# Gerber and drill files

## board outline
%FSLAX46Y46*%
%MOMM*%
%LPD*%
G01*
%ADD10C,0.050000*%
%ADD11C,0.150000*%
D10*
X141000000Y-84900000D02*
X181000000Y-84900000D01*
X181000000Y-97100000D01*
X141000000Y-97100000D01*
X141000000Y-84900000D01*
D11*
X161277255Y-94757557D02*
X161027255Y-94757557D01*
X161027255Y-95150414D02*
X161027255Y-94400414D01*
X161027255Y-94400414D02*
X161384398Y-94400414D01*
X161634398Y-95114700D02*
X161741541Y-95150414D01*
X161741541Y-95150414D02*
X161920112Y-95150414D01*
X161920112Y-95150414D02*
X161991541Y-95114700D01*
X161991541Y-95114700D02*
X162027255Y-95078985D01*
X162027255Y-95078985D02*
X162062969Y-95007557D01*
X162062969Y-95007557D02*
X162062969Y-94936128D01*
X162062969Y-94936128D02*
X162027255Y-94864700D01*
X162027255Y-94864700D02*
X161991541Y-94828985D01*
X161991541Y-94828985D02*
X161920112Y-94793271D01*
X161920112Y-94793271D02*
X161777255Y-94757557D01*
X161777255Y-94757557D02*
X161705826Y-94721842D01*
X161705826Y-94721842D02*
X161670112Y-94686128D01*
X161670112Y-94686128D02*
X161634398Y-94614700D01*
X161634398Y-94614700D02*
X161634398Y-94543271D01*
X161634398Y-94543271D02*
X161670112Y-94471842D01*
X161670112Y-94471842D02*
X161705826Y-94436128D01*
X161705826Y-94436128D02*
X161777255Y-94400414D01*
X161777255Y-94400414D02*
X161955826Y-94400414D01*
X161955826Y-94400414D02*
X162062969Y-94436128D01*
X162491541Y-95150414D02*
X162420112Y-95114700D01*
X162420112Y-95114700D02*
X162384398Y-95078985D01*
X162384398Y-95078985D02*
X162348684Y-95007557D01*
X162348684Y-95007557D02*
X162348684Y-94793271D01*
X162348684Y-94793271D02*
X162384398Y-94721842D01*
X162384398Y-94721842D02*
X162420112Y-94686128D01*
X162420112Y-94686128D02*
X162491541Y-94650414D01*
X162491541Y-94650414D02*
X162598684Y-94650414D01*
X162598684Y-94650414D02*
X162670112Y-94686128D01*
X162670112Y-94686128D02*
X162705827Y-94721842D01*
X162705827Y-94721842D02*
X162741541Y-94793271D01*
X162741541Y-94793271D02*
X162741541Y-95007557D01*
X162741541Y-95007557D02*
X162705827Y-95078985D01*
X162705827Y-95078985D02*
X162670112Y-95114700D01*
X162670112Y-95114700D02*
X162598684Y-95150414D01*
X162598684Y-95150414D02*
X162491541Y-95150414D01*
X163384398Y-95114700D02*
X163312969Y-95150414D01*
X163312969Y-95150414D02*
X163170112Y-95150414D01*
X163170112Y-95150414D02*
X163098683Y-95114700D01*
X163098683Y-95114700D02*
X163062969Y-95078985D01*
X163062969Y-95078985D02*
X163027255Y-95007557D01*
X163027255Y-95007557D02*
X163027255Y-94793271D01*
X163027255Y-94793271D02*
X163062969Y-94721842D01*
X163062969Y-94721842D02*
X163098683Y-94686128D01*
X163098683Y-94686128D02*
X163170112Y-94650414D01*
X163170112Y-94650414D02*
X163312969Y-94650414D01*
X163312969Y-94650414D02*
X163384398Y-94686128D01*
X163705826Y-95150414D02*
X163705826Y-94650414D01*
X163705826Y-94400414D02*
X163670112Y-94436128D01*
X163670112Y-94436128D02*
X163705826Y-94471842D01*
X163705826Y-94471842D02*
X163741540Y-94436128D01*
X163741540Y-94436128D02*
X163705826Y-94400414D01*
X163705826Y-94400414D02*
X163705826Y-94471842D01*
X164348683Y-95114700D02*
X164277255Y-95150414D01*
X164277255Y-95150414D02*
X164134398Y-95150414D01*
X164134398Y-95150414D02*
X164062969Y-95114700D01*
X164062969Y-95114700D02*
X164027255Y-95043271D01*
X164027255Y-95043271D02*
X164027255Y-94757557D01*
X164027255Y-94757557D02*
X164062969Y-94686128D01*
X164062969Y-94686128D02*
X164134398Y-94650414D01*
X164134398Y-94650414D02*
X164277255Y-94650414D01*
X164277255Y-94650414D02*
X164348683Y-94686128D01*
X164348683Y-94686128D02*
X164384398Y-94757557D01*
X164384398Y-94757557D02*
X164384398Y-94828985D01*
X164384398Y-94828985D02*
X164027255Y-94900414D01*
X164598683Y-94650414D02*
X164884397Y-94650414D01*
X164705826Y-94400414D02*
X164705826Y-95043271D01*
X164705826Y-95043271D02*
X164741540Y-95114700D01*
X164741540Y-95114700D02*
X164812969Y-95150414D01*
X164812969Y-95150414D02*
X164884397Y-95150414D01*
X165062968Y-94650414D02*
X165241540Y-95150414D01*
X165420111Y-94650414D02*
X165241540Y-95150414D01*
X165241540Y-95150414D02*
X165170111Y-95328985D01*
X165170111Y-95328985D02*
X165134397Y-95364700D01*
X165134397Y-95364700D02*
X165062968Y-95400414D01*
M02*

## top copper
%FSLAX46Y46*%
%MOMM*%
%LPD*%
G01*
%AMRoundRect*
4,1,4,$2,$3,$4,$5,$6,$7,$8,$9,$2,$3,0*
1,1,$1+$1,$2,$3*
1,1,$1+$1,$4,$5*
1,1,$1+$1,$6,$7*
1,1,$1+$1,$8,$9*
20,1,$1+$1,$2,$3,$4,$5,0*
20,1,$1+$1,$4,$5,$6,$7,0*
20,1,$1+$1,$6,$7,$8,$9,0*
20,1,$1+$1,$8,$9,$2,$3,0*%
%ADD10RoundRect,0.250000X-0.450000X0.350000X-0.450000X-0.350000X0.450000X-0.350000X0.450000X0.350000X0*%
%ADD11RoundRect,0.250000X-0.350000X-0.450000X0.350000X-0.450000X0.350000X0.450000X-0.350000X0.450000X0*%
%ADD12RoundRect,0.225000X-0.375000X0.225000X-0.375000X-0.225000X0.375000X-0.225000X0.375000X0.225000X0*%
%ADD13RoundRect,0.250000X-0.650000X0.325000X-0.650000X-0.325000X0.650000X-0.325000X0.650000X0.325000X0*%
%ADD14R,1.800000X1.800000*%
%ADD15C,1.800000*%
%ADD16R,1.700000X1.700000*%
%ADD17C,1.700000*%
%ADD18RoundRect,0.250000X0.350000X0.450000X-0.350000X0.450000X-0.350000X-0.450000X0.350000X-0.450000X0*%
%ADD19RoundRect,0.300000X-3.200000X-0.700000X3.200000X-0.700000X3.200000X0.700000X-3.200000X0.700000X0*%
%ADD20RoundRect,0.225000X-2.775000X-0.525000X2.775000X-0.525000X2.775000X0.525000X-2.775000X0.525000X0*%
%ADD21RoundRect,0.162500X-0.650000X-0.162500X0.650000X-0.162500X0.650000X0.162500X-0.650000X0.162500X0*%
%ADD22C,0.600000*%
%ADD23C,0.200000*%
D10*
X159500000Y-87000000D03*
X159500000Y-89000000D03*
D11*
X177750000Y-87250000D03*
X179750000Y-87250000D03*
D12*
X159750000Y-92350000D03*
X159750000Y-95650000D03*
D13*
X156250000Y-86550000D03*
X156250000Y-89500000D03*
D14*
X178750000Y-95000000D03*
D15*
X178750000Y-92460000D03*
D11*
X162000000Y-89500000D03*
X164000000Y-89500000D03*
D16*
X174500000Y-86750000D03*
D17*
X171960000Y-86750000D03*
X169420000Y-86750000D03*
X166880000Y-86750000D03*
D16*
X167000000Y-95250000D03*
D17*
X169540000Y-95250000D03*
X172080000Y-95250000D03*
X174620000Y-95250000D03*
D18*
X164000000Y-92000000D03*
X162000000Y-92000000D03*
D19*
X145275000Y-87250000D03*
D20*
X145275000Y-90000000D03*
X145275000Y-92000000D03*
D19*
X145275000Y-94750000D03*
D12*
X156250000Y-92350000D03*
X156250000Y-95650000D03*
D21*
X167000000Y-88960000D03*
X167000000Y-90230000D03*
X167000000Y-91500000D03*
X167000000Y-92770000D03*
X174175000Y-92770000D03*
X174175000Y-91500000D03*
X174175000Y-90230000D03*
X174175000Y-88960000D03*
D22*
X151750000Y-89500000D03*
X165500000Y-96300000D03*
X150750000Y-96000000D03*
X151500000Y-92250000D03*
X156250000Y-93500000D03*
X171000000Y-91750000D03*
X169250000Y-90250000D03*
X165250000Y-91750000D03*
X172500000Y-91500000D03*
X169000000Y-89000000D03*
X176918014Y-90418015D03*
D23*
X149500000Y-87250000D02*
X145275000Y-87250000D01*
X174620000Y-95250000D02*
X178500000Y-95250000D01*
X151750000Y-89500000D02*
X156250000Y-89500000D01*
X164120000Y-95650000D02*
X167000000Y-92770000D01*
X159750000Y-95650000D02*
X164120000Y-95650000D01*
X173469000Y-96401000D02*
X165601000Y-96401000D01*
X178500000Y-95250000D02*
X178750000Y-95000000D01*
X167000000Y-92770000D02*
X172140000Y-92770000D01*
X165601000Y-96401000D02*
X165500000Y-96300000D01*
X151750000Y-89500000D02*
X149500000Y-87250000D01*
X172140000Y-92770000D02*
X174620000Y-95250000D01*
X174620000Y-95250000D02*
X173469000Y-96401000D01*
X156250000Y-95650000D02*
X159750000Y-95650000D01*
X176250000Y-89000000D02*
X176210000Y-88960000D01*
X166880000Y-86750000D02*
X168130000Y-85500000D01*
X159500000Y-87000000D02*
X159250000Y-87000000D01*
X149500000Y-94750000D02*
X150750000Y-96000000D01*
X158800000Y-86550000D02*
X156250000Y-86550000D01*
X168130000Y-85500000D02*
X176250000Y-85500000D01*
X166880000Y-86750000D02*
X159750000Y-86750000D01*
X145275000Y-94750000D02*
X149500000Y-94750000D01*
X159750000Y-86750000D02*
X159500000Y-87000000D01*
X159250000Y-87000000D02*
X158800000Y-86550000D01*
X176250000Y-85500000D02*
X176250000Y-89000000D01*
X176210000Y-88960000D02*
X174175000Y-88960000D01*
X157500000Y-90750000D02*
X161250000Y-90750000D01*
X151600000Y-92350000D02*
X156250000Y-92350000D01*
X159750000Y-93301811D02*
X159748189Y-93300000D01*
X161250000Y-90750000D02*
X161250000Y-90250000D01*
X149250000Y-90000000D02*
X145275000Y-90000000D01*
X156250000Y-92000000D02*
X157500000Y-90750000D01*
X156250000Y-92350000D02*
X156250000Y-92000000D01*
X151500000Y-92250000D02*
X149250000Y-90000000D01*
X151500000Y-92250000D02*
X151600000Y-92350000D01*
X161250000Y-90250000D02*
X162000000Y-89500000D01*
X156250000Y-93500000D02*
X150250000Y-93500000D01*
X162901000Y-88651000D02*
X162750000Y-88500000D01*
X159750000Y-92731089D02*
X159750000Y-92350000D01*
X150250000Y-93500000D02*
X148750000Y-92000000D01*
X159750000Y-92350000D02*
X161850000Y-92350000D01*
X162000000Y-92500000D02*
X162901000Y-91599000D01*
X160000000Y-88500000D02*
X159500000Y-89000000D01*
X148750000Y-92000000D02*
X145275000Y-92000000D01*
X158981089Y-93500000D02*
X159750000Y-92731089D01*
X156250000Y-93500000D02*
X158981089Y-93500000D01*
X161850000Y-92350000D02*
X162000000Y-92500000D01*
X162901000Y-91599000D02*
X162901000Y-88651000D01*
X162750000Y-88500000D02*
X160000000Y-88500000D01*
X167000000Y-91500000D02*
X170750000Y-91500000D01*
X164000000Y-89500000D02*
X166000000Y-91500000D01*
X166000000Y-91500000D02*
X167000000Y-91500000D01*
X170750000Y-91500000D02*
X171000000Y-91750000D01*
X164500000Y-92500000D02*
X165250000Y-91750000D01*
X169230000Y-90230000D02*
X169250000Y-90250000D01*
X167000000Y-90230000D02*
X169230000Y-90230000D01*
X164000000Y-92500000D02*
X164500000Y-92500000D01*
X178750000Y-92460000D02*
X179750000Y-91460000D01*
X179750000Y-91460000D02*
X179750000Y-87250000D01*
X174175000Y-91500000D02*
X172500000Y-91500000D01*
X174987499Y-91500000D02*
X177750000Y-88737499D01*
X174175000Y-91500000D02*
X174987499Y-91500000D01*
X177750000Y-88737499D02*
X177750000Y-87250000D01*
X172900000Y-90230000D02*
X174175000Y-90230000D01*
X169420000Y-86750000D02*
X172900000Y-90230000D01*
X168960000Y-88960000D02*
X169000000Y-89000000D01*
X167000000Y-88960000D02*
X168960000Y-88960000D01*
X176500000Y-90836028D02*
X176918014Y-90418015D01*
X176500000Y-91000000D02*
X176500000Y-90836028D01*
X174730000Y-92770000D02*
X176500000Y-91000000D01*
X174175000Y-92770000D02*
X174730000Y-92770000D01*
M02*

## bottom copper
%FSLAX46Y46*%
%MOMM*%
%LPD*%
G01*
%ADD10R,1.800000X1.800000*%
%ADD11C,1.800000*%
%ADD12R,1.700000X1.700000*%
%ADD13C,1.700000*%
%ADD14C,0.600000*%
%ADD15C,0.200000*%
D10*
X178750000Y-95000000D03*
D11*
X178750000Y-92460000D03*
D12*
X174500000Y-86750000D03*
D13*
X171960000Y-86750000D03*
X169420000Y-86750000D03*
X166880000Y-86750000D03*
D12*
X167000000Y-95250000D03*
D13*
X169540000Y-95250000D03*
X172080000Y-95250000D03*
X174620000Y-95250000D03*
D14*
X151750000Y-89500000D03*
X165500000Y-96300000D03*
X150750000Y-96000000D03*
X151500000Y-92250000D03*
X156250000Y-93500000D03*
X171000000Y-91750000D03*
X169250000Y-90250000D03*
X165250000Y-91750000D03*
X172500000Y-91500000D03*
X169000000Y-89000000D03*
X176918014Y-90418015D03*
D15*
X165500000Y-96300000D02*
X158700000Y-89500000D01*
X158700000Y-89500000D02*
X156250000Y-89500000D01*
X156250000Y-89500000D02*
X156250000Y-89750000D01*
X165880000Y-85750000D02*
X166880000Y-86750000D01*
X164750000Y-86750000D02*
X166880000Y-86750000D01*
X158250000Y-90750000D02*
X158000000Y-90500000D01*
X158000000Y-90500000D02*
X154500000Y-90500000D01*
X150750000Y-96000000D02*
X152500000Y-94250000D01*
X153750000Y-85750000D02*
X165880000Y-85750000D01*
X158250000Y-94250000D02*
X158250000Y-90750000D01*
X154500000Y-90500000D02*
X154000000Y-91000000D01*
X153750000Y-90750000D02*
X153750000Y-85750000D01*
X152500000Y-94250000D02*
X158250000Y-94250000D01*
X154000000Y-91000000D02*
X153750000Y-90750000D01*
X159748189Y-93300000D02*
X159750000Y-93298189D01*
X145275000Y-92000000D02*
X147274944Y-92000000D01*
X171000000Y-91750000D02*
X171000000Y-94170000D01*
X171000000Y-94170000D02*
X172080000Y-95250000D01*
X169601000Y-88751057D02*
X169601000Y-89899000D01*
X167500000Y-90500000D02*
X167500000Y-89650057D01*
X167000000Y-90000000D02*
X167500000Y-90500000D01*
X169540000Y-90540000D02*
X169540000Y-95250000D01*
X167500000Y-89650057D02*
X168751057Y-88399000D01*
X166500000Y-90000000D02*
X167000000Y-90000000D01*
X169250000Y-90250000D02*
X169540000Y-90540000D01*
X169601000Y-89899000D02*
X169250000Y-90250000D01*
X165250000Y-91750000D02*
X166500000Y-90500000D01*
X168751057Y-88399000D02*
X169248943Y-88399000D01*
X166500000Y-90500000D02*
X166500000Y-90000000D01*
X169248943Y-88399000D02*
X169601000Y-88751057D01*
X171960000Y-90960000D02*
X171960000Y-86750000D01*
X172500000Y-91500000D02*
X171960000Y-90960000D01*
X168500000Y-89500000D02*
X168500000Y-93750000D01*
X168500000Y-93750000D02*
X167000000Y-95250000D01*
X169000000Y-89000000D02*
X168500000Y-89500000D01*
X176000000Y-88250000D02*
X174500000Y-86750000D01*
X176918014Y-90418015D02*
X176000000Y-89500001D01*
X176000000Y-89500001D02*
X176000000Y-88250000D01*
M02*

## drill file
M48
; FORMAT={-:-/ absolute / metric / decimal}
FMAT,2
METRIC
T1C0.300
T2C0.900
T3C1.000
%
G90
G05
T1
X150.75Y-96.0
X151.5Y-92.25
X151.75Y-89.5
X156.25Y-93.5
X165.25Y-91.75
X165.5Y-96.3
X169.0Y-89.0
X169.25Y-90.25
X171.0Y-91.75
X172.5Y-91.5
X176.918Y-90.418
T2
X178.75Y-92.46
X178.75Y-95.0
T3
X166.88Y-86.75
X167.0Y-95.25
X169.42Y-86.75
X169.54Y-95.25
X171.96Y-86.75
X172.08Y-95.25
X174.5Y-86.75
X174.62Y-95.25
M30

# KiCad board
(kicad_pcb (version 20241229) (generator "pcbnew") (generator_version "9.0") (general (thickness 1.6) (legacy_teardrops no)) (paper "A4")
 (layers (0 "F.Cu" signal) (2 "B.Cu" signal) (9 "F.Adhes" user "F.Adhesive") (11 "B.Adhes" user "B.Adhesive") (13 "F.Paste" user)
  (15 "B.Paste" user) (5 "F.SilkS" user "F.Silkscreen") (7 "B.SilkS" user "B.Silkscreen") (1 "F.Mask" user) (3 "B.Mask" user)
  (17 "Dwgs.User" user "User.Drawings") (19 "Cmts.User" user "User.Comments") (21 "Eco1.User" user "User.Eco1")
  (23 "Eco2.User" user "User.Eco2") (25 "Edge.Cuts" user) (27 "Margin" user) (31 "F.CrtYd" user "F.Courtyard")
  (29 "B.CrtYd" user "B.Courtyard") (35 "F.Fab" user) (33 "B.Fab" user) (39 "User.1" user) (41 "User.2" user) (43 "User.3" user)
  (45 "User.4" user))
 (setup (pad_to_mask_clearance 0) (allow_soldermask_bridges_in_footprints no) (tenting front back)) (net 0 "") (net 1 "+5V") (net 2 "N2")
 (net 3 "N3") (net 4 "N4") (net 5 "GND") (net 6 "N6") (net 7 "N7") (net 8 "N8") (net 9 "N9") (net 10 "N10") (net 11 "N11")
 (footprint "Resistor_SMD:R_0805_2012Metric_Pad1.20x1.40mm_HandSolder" (layer "F.Cu") (at 159.5 88 -90)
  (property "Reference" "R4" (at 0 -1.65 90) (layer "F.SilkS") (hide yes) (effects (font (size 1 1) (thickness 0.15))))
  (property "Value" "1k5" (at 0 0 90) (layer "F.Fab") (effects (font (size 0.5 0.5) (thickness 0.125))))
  (pad "1" smd roundrect (at -1 0 270) (size 1.2 1.4) (layers "F.Cu" "F.Mask" "F.Paste") (roundrect_rratio 0.208333) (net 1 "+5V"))
  (pad "2" smd roundrect (at 1 0 270) (size 1.2 1.4) (layers "F.Cu" "F.Mask" "F.Paste") (roundrect_rratio 0.208333) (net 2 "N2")))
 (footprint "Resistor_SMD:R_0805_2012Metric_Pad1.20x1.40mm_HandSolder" (layer "F.Cu") (at 178.75 87.25)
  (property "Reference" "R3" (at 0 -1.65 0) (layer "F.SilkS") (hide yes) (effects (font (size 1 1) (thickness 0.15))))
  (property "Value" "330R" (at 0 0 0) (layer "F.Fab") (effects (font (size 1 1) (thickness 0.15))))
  (pad "1" smd roundrect (at -1 0) (size 1.2 1.4) (layers "F.Cu" "F.Mask" "F.Paste") (roundrect_rratio 0.208333) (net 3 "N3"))
  (pad "2" smd roundrect (at 1 0) (size 1.2 1.4) (layers "F.Cu" "F.Mask" "F.Paste") (roundrect_rratio 0.208333) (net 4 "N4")))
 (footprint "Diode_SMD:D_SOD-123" (layer "F.Cu") (at 159.75 94 -90)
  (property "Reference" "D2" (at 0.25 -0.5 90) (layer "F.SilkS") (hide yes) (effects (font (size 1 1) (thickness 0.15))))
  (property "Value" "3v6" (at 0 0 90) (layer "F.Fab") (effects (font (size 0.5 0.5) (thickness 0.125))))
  (pad "1" smd roundrect (at -1.65 0 270) (size 0.9 1.2) (layers "F.Cu" "F.Mask" "F.Paste") (roundrect_rratio 0.25) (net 2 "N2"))
  (pad "2" smd roundrect (at 1.65 0 270) (size 0.9 1.2) (layers "F.Cu" "F.Mask" "F.Paste") (roundrect_rratio 0.25) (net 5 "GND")))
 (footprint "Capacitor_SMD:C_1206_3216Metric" (layer "F.Cu") (at 156.25 88.025 -90)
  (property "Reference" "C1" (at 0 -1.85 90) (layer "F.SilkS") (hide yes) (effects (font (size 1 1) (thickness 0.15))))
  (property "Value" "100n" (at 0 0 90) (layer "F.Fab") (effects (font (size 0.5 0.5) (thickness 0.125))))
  (pad "1" smd roundrect (at -1.475 0 270) (size 1.15 1.8) (layers "F.Cu" "F.Mask" "F.Paste") (roundrect_rratio 0.217391) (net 1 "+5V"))
  (pad "2" smd roundrect (at 1.475 0 270) (size 1.15 1.8) (layers "F.Cu" "F.Mask" "F.Paste") (roundrect_rratio 0.217391) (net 5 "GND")))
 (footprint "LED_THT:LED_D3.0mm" (layer "F.Cu") (at 178.75 95 90)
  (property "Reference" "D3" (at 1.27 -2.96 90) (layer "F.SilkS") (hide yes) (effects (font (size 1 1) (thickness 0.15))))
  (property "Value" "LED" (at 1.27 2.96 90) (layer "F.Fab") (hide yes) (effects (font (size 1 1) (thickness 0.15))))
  (pad "1" thru_hole rect (at 0 0 90) (size 1.8 1.8) (drill 0.9) (layers "*.Cu" "*.Mask") (remove_unused_layers no) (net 5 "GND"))
  (pad "2" thru_hole circle (at 2.54 0 90) (size 1.8 1.8) (drill 0.9) (layers "*.Cu" "*.Mask") (remove_unused_layers no) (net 4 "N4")))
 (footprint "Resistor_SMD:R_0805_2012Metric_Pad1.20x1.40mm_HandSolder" (layer "F.Cu") (at 163 89.5)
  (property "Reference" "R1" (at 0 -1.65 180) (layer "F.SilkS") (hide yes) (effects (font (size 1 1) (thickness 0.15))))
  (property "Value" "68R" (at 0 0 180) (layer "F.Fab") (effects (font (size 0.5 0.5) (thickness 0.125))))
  (pad "1" smd roundrect (at -1 0) (size 1.2 1.4) (layers "F.Cu" "F.Mask" "F.Paste") (roundrect_rratio 0.208333) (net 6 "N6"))
  (pad "2" smd roundrect (at 1 0) (size 1.2 1.4) (layers "F.Cu" "F.Mask" "F.Paste") (roundrect_rratio 0.208333) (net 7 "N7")))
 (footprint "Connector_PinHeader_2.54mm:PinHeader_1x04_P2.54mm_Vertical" (layer "F.Cu") (at 174.5 86.75 -90)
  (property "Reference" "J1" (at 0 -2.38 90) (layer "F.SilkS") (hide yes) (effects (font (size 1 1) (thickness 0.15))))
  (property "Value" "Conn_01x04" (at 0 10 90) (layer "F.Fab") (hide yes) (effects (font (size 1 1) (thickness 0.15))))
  (pad "1" thru_hole rect (at 0 0 270) (size 1.7 1.7) (drill 1) (layers "*.Cu" "*.Mask") (remove_unused_layers no) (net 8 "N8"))
  (pad "2" thru_hole circle (at 0 2.54 270) (size 1.7 1.7) (drill 1) (layers "*.Cu" "*.Mask") (remove_unused_layers no) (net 3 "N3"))
  (pad "3" thru_hole circle (at 0 5.08 270) (size 1.7 1.7) (drill 1) (layers "*.Cu" "*.Mask") (remove_unused_layers no) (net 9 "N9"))
  (pad "4" thru_hole circle (at 0 7.62 270) (size 1.7 1.7) (drill 1) (layers "*.Cu" "*.Mask") (remove_unused_layers no) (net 1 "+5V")))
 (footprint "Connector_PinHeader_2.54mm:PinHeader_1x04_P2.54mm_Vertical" (layer "F.Cu") (at 167 95.25 90)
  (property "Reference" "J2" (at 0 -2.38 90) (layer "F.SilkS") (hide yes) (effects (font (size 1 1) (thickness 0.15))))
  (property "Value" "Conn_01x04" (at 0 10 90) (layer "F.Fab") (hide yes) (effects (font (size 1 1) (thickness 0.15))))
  (pad "1" thru_hole rect (at 0 0 90) (size 1.7 1.7) (drill 1) (layers "*.Cu" "*.Mask") (remove_unused_layers no) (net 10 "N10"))
  (pad "2" thru_hole circle (at 0 2.54 90) (size 1.7 1.7) (drill 1) (layers "*.Cu" "*.Mask") (remove_unused_layers no) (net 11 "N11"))
  (pad "3" thru_hole circle (at 0 5.08 90) (size 1.7 1.7) (drill 1) (layers "*.Cu" "*.Mask") (remove_unused_layers no) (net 7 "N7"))
  (pad "4" thru_hole circle (at 0 7.62 90) (size 1.7 1.7) (drill 1) (layers "*.Cu" "*.Mask") (remove_unused_layers no) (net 5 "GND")))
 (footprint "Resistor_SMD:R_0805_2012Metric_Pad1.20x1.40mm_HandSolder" (layer "F.Cu") (at 163 92 180)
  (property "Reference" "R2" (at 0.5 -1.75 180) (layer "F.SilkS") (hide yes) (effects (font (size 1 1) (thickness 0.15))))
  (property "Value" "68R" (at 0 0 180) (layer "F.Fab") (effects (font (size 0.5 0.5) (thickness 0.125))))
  (pad "1" smd roundrect (at -1 0 180) (size 1.2 1.4) (layers "F.Cu" "F.Mask" "F.Paste") (roundrect_rratio 0.208333) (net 11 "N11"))
  (pad "2" smd roundrect (at 1 0 180) (size 1.2 1.4) (layers "F.Cu" "F.Mask" "F.Paste") (roundrect_rratio 0.208333) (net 2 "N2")))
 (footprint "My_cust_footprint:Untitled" (layer "F.Cu") (at 145.275 91)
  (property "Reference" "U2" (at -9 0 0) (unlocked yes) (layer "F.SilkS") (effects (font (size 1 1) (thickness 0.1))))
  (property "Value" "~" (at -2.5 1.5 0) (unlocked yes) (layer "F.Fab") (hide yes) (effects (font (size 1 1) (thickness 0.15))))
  (pad "1" smd roundrect (at 0 -3.75) (size 7 2) (layers "F.Cu" "F.Mask" "F.Paste") (roundrect_rratio 0.15) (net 5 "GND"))
  (pad "2" smd roundrect (at 0 -1) (size 6 1.5) (layers "F.Cu" "F.Mask" "F.Paste") (roundrect_rratio 0.15) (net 6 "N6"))
  (pad "3" smd roundrect (at 0 1) (size 6 1.5) (layers "F.Cu" "F.Mask" "F.Paste") (roundrect_rratio 0.15) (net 2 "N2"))
  (pad "4" smd roundrect (at 0 3.75) (size 7 2) (layers "F.Cu" "F.Mask" "F.Paste") (roundrect_rratio 0.15) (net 1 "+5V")))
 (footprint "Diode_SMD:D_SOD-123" (layer "F.Cu") (at 156.25 94 -90)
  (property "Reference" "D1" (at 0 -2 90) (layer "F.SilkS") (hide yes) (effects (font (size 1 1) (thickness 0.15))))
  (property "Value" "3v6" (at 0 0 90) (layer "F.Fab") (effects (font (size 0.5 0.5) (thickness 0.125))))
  (pad "1" smd roundrect (at -1.65 0 270) (size 0.9 1.2) (layers "F.Cu" "F.Mask" "F.Paste") (roundrect_rratio 0.25) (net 6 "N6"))
  (pad "2" smd roundrect (at 1.65 0 270) (size 0.9 1.2) (layers "F.Cu" "F.Mask" "F.Paste") (roundrect_rratio 0.25) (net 5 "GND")))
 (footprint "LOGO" (layer "F.Cu") (at 152 91.5)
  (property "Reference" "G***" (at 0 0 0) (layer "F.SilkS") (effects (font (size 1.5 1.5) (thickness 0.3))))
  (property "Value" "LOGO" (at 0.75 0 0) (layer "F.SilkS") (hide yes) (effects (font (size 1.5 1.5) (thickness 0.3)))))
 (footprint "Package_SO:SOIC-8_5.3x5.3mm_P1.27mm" (layer "F.Cu") (at 170.5875 90.865)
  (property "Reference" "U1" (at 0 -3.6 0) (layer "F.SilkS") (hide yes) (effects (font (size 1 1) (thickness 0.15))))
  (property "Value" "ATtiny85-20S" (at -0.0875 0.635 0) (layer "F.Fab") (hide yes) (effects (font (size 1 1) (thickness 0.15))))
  (pad "1" smd roundrect (at -3.5875 -1.905) (size 1.625 0.65) (layers "F.Cu" "F.Mask" "F.Paste") (roundrect_rratio 0.25) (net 10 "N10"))
  (pad "2" smd roundrect (at -3.5875 -0.635) (size 1.625 0.65) (layers "F.Cu" "F.Mask" "F.Paste") (roundrect_rratio 0.25) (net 11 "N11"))
  (pad "3" smd roundrect (at -3.5875 0.635) (size 1.625 0.65) (layers "F.Cu" "F.Mask" "F.Paste") (roundrect_rratio 0.25) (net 7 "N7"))
  (pad "4" smd roundrect (at -3.5875 1.905) (size 1.625 0.65) (layers "F.Cu" "F.Mask" "F.Paste") (roundrect_rratio 0.25) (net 5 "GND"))
  (pad "5" smd roundrect (at 3.5875 1.905) (size 1.625 0.65) (layers "F.Cu" "F.Mask" "F.Paste") (roundrect_rratio 0.25) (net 8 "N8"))
  (pad "6" smd roundrect (at 3.5875 0.635) (size 1.625 0.65) (layers "F.Cu" "F.Mask" "F.Paste") (roundrect_rratio 0.25) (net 3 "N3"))
  (pad "7" smd roundrect (at 3.5875 -0.635) (size 1.625 0.65) (layers "F.Cu" "F.Mask" "F.Paste") (roundrect_rratio 0.25) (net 9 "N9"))
  (pad "8" smd roundrect (at 3.5875 -1.905) (size 1.625 0.65) (layers "F.Cu" "F.Mask" "F.Paste") (roundrect_rratio 0.25) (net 1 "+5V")))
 (gr_rect (start 141 84.9) (end 181 97.1) (stroke (width 0.05) (type solid)) (fill no) (layer "Edge.Cuts"))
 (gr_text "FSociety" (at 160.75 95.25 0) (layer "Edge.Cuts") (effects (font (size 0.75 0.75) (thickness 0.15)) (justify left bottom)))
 (segment (start 149.5 87.25) (end 145.275 87.25) (width 0.2) (layer "F.Cu") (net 5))
 (segment (start 174.62 95.25) (end 178.5 95.25) (width 0.2) (layer "F.Cu") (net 5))
 (segment (start 151.75 89.5) (end 156.25 89.5) (width 0.2) (layer "F.Cu") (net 5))
 (segment (start 164.12 95.65) (end 167 92.77) (width 0.2) (layer "F.Cu") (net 5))
 (segment (start 159.75 95.65) (end 164.12 95.65) (width 0.2) (layer "F.Cu") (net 5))
 (segment (start 173.469 96.401) (end 165.601 96.401) (width 0.2) (layer "F.Cu") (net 5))
 (segment (start 178.5 95.25) (end 178.75 95) (width 0.2) (layer "F.Cu") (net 5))
 (segment (start 167 92.77) (end 172.14 92.77) (width 0.2) (layer "F.Cu") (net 5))
 (segment (start 165.601 96.401) (end 165.5 96.3) (width 0.2) (layer "F.Cu") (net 5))
 (segment (start 151.75 89.5) (end 149.5 87.25) (width 0.2) (layer "F.Cu") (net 5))
 (segment (start 172.14 92.77) (end 174.62 95.25) (width 0.2) (layer "F.Cu") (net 5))
 (segment (start 174.62 95.25) (end 173.469 96.401) (width 0.2) (layer "F.Cu") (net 5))
 (segment (start 156.25 95.65) (end 159.75 95.65) (width 0.2) (layer "F.Cu") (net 5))
 (via (at 151.75 89.5) (size 0.6) (drill 0.3) (layers "F.Cu" "B.Cu") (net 5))
 (via (at 165.5 96.3) (size 0.6) (drill 0.3) (layers "F.Cu" "B.Cu") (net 5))
 (segment (start 165.5 96.3) (end 158.7 89.5) (width 0.2) (layer "B.Cu") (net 5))
 (segment (start 158.7 89.5) (end 156.25 89.5) (width 0.2) (layer "B.Cu") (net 5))
 (segment (start 156.25 89.5) (end 156.25 89.75) (width 0.2) (layer "B.Cu") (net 5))
 (segment (start 176.25 89) (end 176.21 88.96) (width 0.2) (layer "F.Cu") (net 1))
 (segment (start 166.88 86.75) (end 168.13 85.5) (width 0.2) (layer "F.Cu") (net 1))
 (segment (start 159.5 87) (end 159.25 87) (width 0.2) (layer "F.Cu") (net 1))
 (segment (start 149.5 94.75) (end 150.75 96) (width 0.2) (layer "F.Cu") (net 1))
 (segment (start 158.8 86.55) (end 156.25 86.55) (width 0.2) (layer "F.Cu") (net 1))
 (segment (start 168.13 85.5) (end 176.25 85.5) (width 0.2) (layer "F.Cu") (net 1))
 (segment (start 166.88 86.75) (end 159.75 86.75) (width 0.2) (layer "F.Cu") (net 1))
 (segment (start 145.275 94.75) (end 149.5 94.75) (width 0.2) (layer "F.Cu") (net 1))
 (segment (start 159.75 86.75) (end 159.5 87) (width 0.2) (layer "F.Cu") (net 1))
 (segment (start 159.25 87) (end 158.8 86.55) (width 0.2) (layer "F.Cu") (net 1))
 (segment (start 176.25 85.5) (end 176.25 89) (width 0.2) (layer "F.Cu") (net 1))
 (segment (start 176.21 88.96) (end 174.175 88.96) (width 0.2) (layer "F.Cu") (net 1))
 (via (at 150.75 96) (size 0.6) (drill 0.3) (layers "F.Cu" "B.Cu") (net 1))
 (segment (start 165.88 85.75) (end 166.88 86.75) (width 0.2) (layer "B.Cu") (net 1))
 (segment (start 164.75 86.75) (end 166.88 86.75) (width 0.2) (layer "B.Cu") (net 1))
 (segment (start 158.25 90.75) (end 158 90.5) (width 0.2) (layer "B.Cu") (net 1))
 (segment (start 158 90.5) (end 154.5 90.5) (width 0.2) (layer "B.Cu") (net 1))
 (segment (start 150.75 96) (end 152.5 94.25) (width 0.2) (layer "B.Cu") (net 1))
 (segment (start 153.75 85.75) (end 165.88 85.75) (width 0.2) (layer "B.Cu") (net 1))
 (segment (start 158.25 94.25) (end 158.25 90.75) (width 0.2) (layer "B.Cu") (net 1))
 (segment (start 154.5 90.5) (end 154 91) (width 0.2) (layer "B.Cu") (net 1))
 (segment (start 153.75 90.75) (end 153.75 85.75) (width 0.2) (layer "B.Cu") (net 1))
 (segment (start 152.5 94.25) (end 158.25 94.25) (width 0.2) (layer "B.Cu") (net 1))
 (segment (start 154 91) (end 153.75 90.75) (width 0.2) (layer "B.Cu") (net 1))
 (segment (start 157.5 90.75) (end 161.25 90.75) (width 0.2) (layer "F.Cu") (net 6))
 (segment (start 151.6 92.35) (end 156.25 92.35) (width 0.2) (layer "F.Cu") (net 6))
 (segment (start 159.75 93.301811) (end 159.748189 93.3) (width 0.2) (layer "F.Cu") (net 6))
 (segment (start 161.25 90.75) (end 161.25 90.25) (width 0.2) (layer "F.Cu") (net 6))
 (segment (start 149.25 90) (end 145.275 90) (width 0.2) (layer "F.Cu") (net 6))
 (segment (start 156.25 92) (end 157.5 90.75) (width 0.2) (layer "F.Cu") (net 6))
 (segment (start 156.25 92.35) (end 156.25 92) (width 0.2) (layer "F.Cu") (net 6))
 (segment (start 151.5 92.25) (end 149.25 90) (width 0.2) (layer "F.Cu") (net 6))
 (segment (start 151.5 92.25) (end 151.6 92.35) (width 0.2) (layer "F.Cu") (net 6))
 (segment (start 161.25 90.25) (end 162 89.5) (width 0.2) (layer "F.Cu") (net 6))
 (via (at 151.5 92.25) (size 0.6) (drill 0.3) (layers "F.Cu" "B.Cu") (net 6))
 (segment (start 159.748189 93.3) (end 159.75 93.298189) (width 0.2) (layer "B.Cu") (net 6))
 (segment (start 156.25 93.5) (end 150.25 93.5) (width 0.2) (layer "F.Cu") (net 2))
 (segment (start 162.901 88.651) (end 162.75 88.5) (width 0.2) (layer "F.Cu") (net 2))
 (segment (start 159.75 92.731089) (end 159.75 92.35) (width 0.2) (layer "F.Cu") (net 2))
 (segment (start 150.25 93.5) (end 148.75 92) (width 0.2) (layer "F.Cu") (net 2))
 (segment (start 159.75 92.35) (end 161.85 92.35) (width 0.2) (layer "F.Cu") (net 2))
 (segment (start 162 92.5) (end 162.901 91.599) (width 0.2) (layer "F.Cu") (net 2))
 (segment (start 160 88.5) (end 159.5 89) (width 0.2) (layer "F.Cu") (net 2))
 (segment (start 148.75 92) (end 145.275 92) (width 0.2) (layer "F.Cu") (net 2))
 (segment (start 158.981089 93.5) (end 159.75 92.731089) (width 0.2) (layer "F.Cu") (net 2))
 (segment (start 156.25 93.5) (end 158.981089 93.5) (width 0.2) (layer "F.Cu") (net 2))
 (segment (start 161.85 92.35) (end 162 92.5) (width 0.2) (layer "F.Cu") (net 2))
 (segment (start 162.901 91.599) (end 162.901 88.651) (width 0.2) (layer "F.Cu") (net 2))
 (segment (start 162.75 88.5) (end 160 88.5) (width 0.2) (layer "F.Cu") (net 2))
 (via (at 156.25 93.5) (size 0.6) (drill 0.3) (layers "F.Cu" "B.Cu") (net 2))
 (segment (start 145.275 92) (end 147.274944 92) (width 0.2) (layer "B.Cu") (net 2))
 (segment (start 167 91.5) (end 170.75 91.5) (width 0.2) (layer "F.Cu") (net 7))
 (segment (start 164 89.5) (end 166 91.5) (width 0.2) (layer "F.Cu") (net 7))
 (segment (start 166 91.5) (end 167 91.5) (width 0.2) (layer "F.Cu") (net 7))
 (segment (start 170.75 91.5) (end 171 91.75) (width 0.2) (layer "F.Cu") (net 7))
 (via (at 171 91.75) (size 0.6) (drill 0.3) (layers "F.Cu" "B.Cu") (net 7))
 (segment (start 171 91.75) (end 171 94.17) (width 0.2) (layer "B.Cu") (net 7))
 (segment (start 171 94.17) (end 172.08 95.25) (width 0.2) (layer "B.Cu") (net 7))
 (segment (start 164.5 92.5) (end 165.25 91.75) (width 0.2) (layer "F.Cu") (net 11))
 (segment (start 169.23 90.23) (end 169.25 90.25) (width 0.2) (layer "F.Cu") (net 11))
 (segment (start 167 90.23) (end 169.23 90.23) (width 0.2) (layer "F.Cu") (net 11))
 (segment (start 164 92.5) (end 164.5 92.5) (width 0.2) (layer "F.Cu") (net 11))
 (via (at 169.25 90.25) (size 0.6) (drill 0.3) (layers "F.Cu" "B.Cu") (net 11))
 (via (at 165.25 91.75) (size 0.6) (drill 0.3) (layers "F.Cu" "B.Cu") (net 11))
 (segment (start 169.601 88.751057) (end 169.601 89.899) (width 0.2) (layer "B.Cu") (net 11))
 (segment (start 167.5 90.5) (end 167.5 89.650057) (width 0.2) (layer "B.Cu") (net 11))
 (segment (start 167 90) (end 167.5 90.5) (width 0.2) (layer "B.Cu") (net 11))
 (segment (start 169.54 90.54) (end 169.54 95.25) (width 0.2) (layer "B.Cu") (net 11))
 (segment (start 167.5 89.650057) (end 168.751057 88.399) (width 0.2) (layer "B.Cu") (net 11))
 (segment (start 166.5 90) (end 167 90) (width 0.2) (layer "B.Cu") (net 11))
 (segment (start 169.25 90.25) (end 169.54 90.54) (width 0.2) (layer "B.Cu") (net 11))
 (segment (start 169.601 89.899) (end 169.25 90.25) (width 0.2) (layer "B.Cu") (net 11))
 (segment (start 165.25 91.75) (end 166.5 90.5) (width 0.2) (layer "B.Cu") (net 11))
 (segment (start 168.751057 88.399) (end 169.248943 88.399) (width 0.2) (layer "B.Cu") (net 11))
 (segment (start 166.5 90.5) (end 166.5 90) (width 0.2) (layer "B.Cu") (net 11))
 (segment (start 169.248943 88.399) (end 169.601 88.751057) (width 0.2) (layer "B.Cu") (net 11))
 (segment (start 178.75 92.46) (end 179.75 91.46) (width 0.2) (layer "F.Cu") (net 4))
 (segment (start 179.75 91.46) (end 179.75 87.25) (width 0.2) (layer "F.Cu") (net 4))
 (segment (start 174.175 91.5) (end 172.5 91.5) (width 0.2) (layer "F.Cu") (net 3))
 (segment (start 174.987499 91.5) (end 177.75 88.737499) (width 0.2) (layer "F.Cu") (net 3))
 (segment (start 174.175 91.5) (end 174.987499 91.5) (width 0.2) (layer "F.Cu") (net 3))
 (segment (start 177.75 88.737499) (end 177.75 87.25) (width 0.2) (layer "F.Cu") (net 3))
 (via (at 172.5 91.5) (size 0.6) (drill 0.3) (layers "F.Cu" "B.Cu") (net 3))
 (segment (start 171.96 90.96) (end 171.96 86.75) (width 0.2) (layer "B.Cu") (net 3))
 (segment (start 172.5 91.5) (end 171.96 90.96) (width 0.2) (layer "B.Cu") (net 3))
 (segment (start 172.9 90.23) (end 174.175 90.23) (width 0.2) (layer "F.Cu") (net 9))
 (segment (start 169.42 86.75) (end 172.9 90.23) (width 0.2) (layer "F.Cu") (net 9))
 (segment (start 168.96 88.96) (end 169 89) (width 0.2) (layer "F.Cu") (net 10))
 (segment (start 167 88.96) (end 168.96 88.96) (width 0.2) (layer "F.Cu") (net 10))
 (via (at 169 89) (size 0.6) (drill 0.3) (layers "F.Cu" "B.Cu") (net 10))
 (segment (start 168.5 89.5) (end 168.5 93.75) (width 0.2) (layer "B.Cu") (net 10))
 (segment (start 168.5 93.75) (end 167 95.25) (width 0.2) (layer "B.Cu") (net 10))
 (segment (start 169 89) (end 168.5 89.5) (width 0.2) (layer "B.Cu") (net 10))
 (segment (start 176.5 90.836028) (end 176.918014 90.418015) (width 0.2) (layer "F.Cu") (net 8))
 (segment (start 176.5 91) (end 176.5 90.836028) (width 0.2) (layer "F.Cu") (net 8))
 (segment (start 174.73 92.77) (end 176.5 91) (width 0.2) (layer "F.Cu") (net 8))
 (segment (start 174.175 92.77) (end 174.73 92.77) (width 0.2) (layer "F.Cu") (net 8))
 (via (at 176.918014 90.418015) (size 0.6) (drill 0.3) (layers "F.Cu" "B.Cu") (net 8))
 (segment (start 176 88.25) (end 174.5 86.75) (width 0.2) (layer "B.Cu") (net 8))
 (segment (start 176.918014 90.418015) (end 176 89.500001) (width 0.2) (layer "B.Cu") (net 8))
 (segment (start 176 89.500001) (end 176 88.25) (width 0.2) (layer "B.Cu") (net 8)))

